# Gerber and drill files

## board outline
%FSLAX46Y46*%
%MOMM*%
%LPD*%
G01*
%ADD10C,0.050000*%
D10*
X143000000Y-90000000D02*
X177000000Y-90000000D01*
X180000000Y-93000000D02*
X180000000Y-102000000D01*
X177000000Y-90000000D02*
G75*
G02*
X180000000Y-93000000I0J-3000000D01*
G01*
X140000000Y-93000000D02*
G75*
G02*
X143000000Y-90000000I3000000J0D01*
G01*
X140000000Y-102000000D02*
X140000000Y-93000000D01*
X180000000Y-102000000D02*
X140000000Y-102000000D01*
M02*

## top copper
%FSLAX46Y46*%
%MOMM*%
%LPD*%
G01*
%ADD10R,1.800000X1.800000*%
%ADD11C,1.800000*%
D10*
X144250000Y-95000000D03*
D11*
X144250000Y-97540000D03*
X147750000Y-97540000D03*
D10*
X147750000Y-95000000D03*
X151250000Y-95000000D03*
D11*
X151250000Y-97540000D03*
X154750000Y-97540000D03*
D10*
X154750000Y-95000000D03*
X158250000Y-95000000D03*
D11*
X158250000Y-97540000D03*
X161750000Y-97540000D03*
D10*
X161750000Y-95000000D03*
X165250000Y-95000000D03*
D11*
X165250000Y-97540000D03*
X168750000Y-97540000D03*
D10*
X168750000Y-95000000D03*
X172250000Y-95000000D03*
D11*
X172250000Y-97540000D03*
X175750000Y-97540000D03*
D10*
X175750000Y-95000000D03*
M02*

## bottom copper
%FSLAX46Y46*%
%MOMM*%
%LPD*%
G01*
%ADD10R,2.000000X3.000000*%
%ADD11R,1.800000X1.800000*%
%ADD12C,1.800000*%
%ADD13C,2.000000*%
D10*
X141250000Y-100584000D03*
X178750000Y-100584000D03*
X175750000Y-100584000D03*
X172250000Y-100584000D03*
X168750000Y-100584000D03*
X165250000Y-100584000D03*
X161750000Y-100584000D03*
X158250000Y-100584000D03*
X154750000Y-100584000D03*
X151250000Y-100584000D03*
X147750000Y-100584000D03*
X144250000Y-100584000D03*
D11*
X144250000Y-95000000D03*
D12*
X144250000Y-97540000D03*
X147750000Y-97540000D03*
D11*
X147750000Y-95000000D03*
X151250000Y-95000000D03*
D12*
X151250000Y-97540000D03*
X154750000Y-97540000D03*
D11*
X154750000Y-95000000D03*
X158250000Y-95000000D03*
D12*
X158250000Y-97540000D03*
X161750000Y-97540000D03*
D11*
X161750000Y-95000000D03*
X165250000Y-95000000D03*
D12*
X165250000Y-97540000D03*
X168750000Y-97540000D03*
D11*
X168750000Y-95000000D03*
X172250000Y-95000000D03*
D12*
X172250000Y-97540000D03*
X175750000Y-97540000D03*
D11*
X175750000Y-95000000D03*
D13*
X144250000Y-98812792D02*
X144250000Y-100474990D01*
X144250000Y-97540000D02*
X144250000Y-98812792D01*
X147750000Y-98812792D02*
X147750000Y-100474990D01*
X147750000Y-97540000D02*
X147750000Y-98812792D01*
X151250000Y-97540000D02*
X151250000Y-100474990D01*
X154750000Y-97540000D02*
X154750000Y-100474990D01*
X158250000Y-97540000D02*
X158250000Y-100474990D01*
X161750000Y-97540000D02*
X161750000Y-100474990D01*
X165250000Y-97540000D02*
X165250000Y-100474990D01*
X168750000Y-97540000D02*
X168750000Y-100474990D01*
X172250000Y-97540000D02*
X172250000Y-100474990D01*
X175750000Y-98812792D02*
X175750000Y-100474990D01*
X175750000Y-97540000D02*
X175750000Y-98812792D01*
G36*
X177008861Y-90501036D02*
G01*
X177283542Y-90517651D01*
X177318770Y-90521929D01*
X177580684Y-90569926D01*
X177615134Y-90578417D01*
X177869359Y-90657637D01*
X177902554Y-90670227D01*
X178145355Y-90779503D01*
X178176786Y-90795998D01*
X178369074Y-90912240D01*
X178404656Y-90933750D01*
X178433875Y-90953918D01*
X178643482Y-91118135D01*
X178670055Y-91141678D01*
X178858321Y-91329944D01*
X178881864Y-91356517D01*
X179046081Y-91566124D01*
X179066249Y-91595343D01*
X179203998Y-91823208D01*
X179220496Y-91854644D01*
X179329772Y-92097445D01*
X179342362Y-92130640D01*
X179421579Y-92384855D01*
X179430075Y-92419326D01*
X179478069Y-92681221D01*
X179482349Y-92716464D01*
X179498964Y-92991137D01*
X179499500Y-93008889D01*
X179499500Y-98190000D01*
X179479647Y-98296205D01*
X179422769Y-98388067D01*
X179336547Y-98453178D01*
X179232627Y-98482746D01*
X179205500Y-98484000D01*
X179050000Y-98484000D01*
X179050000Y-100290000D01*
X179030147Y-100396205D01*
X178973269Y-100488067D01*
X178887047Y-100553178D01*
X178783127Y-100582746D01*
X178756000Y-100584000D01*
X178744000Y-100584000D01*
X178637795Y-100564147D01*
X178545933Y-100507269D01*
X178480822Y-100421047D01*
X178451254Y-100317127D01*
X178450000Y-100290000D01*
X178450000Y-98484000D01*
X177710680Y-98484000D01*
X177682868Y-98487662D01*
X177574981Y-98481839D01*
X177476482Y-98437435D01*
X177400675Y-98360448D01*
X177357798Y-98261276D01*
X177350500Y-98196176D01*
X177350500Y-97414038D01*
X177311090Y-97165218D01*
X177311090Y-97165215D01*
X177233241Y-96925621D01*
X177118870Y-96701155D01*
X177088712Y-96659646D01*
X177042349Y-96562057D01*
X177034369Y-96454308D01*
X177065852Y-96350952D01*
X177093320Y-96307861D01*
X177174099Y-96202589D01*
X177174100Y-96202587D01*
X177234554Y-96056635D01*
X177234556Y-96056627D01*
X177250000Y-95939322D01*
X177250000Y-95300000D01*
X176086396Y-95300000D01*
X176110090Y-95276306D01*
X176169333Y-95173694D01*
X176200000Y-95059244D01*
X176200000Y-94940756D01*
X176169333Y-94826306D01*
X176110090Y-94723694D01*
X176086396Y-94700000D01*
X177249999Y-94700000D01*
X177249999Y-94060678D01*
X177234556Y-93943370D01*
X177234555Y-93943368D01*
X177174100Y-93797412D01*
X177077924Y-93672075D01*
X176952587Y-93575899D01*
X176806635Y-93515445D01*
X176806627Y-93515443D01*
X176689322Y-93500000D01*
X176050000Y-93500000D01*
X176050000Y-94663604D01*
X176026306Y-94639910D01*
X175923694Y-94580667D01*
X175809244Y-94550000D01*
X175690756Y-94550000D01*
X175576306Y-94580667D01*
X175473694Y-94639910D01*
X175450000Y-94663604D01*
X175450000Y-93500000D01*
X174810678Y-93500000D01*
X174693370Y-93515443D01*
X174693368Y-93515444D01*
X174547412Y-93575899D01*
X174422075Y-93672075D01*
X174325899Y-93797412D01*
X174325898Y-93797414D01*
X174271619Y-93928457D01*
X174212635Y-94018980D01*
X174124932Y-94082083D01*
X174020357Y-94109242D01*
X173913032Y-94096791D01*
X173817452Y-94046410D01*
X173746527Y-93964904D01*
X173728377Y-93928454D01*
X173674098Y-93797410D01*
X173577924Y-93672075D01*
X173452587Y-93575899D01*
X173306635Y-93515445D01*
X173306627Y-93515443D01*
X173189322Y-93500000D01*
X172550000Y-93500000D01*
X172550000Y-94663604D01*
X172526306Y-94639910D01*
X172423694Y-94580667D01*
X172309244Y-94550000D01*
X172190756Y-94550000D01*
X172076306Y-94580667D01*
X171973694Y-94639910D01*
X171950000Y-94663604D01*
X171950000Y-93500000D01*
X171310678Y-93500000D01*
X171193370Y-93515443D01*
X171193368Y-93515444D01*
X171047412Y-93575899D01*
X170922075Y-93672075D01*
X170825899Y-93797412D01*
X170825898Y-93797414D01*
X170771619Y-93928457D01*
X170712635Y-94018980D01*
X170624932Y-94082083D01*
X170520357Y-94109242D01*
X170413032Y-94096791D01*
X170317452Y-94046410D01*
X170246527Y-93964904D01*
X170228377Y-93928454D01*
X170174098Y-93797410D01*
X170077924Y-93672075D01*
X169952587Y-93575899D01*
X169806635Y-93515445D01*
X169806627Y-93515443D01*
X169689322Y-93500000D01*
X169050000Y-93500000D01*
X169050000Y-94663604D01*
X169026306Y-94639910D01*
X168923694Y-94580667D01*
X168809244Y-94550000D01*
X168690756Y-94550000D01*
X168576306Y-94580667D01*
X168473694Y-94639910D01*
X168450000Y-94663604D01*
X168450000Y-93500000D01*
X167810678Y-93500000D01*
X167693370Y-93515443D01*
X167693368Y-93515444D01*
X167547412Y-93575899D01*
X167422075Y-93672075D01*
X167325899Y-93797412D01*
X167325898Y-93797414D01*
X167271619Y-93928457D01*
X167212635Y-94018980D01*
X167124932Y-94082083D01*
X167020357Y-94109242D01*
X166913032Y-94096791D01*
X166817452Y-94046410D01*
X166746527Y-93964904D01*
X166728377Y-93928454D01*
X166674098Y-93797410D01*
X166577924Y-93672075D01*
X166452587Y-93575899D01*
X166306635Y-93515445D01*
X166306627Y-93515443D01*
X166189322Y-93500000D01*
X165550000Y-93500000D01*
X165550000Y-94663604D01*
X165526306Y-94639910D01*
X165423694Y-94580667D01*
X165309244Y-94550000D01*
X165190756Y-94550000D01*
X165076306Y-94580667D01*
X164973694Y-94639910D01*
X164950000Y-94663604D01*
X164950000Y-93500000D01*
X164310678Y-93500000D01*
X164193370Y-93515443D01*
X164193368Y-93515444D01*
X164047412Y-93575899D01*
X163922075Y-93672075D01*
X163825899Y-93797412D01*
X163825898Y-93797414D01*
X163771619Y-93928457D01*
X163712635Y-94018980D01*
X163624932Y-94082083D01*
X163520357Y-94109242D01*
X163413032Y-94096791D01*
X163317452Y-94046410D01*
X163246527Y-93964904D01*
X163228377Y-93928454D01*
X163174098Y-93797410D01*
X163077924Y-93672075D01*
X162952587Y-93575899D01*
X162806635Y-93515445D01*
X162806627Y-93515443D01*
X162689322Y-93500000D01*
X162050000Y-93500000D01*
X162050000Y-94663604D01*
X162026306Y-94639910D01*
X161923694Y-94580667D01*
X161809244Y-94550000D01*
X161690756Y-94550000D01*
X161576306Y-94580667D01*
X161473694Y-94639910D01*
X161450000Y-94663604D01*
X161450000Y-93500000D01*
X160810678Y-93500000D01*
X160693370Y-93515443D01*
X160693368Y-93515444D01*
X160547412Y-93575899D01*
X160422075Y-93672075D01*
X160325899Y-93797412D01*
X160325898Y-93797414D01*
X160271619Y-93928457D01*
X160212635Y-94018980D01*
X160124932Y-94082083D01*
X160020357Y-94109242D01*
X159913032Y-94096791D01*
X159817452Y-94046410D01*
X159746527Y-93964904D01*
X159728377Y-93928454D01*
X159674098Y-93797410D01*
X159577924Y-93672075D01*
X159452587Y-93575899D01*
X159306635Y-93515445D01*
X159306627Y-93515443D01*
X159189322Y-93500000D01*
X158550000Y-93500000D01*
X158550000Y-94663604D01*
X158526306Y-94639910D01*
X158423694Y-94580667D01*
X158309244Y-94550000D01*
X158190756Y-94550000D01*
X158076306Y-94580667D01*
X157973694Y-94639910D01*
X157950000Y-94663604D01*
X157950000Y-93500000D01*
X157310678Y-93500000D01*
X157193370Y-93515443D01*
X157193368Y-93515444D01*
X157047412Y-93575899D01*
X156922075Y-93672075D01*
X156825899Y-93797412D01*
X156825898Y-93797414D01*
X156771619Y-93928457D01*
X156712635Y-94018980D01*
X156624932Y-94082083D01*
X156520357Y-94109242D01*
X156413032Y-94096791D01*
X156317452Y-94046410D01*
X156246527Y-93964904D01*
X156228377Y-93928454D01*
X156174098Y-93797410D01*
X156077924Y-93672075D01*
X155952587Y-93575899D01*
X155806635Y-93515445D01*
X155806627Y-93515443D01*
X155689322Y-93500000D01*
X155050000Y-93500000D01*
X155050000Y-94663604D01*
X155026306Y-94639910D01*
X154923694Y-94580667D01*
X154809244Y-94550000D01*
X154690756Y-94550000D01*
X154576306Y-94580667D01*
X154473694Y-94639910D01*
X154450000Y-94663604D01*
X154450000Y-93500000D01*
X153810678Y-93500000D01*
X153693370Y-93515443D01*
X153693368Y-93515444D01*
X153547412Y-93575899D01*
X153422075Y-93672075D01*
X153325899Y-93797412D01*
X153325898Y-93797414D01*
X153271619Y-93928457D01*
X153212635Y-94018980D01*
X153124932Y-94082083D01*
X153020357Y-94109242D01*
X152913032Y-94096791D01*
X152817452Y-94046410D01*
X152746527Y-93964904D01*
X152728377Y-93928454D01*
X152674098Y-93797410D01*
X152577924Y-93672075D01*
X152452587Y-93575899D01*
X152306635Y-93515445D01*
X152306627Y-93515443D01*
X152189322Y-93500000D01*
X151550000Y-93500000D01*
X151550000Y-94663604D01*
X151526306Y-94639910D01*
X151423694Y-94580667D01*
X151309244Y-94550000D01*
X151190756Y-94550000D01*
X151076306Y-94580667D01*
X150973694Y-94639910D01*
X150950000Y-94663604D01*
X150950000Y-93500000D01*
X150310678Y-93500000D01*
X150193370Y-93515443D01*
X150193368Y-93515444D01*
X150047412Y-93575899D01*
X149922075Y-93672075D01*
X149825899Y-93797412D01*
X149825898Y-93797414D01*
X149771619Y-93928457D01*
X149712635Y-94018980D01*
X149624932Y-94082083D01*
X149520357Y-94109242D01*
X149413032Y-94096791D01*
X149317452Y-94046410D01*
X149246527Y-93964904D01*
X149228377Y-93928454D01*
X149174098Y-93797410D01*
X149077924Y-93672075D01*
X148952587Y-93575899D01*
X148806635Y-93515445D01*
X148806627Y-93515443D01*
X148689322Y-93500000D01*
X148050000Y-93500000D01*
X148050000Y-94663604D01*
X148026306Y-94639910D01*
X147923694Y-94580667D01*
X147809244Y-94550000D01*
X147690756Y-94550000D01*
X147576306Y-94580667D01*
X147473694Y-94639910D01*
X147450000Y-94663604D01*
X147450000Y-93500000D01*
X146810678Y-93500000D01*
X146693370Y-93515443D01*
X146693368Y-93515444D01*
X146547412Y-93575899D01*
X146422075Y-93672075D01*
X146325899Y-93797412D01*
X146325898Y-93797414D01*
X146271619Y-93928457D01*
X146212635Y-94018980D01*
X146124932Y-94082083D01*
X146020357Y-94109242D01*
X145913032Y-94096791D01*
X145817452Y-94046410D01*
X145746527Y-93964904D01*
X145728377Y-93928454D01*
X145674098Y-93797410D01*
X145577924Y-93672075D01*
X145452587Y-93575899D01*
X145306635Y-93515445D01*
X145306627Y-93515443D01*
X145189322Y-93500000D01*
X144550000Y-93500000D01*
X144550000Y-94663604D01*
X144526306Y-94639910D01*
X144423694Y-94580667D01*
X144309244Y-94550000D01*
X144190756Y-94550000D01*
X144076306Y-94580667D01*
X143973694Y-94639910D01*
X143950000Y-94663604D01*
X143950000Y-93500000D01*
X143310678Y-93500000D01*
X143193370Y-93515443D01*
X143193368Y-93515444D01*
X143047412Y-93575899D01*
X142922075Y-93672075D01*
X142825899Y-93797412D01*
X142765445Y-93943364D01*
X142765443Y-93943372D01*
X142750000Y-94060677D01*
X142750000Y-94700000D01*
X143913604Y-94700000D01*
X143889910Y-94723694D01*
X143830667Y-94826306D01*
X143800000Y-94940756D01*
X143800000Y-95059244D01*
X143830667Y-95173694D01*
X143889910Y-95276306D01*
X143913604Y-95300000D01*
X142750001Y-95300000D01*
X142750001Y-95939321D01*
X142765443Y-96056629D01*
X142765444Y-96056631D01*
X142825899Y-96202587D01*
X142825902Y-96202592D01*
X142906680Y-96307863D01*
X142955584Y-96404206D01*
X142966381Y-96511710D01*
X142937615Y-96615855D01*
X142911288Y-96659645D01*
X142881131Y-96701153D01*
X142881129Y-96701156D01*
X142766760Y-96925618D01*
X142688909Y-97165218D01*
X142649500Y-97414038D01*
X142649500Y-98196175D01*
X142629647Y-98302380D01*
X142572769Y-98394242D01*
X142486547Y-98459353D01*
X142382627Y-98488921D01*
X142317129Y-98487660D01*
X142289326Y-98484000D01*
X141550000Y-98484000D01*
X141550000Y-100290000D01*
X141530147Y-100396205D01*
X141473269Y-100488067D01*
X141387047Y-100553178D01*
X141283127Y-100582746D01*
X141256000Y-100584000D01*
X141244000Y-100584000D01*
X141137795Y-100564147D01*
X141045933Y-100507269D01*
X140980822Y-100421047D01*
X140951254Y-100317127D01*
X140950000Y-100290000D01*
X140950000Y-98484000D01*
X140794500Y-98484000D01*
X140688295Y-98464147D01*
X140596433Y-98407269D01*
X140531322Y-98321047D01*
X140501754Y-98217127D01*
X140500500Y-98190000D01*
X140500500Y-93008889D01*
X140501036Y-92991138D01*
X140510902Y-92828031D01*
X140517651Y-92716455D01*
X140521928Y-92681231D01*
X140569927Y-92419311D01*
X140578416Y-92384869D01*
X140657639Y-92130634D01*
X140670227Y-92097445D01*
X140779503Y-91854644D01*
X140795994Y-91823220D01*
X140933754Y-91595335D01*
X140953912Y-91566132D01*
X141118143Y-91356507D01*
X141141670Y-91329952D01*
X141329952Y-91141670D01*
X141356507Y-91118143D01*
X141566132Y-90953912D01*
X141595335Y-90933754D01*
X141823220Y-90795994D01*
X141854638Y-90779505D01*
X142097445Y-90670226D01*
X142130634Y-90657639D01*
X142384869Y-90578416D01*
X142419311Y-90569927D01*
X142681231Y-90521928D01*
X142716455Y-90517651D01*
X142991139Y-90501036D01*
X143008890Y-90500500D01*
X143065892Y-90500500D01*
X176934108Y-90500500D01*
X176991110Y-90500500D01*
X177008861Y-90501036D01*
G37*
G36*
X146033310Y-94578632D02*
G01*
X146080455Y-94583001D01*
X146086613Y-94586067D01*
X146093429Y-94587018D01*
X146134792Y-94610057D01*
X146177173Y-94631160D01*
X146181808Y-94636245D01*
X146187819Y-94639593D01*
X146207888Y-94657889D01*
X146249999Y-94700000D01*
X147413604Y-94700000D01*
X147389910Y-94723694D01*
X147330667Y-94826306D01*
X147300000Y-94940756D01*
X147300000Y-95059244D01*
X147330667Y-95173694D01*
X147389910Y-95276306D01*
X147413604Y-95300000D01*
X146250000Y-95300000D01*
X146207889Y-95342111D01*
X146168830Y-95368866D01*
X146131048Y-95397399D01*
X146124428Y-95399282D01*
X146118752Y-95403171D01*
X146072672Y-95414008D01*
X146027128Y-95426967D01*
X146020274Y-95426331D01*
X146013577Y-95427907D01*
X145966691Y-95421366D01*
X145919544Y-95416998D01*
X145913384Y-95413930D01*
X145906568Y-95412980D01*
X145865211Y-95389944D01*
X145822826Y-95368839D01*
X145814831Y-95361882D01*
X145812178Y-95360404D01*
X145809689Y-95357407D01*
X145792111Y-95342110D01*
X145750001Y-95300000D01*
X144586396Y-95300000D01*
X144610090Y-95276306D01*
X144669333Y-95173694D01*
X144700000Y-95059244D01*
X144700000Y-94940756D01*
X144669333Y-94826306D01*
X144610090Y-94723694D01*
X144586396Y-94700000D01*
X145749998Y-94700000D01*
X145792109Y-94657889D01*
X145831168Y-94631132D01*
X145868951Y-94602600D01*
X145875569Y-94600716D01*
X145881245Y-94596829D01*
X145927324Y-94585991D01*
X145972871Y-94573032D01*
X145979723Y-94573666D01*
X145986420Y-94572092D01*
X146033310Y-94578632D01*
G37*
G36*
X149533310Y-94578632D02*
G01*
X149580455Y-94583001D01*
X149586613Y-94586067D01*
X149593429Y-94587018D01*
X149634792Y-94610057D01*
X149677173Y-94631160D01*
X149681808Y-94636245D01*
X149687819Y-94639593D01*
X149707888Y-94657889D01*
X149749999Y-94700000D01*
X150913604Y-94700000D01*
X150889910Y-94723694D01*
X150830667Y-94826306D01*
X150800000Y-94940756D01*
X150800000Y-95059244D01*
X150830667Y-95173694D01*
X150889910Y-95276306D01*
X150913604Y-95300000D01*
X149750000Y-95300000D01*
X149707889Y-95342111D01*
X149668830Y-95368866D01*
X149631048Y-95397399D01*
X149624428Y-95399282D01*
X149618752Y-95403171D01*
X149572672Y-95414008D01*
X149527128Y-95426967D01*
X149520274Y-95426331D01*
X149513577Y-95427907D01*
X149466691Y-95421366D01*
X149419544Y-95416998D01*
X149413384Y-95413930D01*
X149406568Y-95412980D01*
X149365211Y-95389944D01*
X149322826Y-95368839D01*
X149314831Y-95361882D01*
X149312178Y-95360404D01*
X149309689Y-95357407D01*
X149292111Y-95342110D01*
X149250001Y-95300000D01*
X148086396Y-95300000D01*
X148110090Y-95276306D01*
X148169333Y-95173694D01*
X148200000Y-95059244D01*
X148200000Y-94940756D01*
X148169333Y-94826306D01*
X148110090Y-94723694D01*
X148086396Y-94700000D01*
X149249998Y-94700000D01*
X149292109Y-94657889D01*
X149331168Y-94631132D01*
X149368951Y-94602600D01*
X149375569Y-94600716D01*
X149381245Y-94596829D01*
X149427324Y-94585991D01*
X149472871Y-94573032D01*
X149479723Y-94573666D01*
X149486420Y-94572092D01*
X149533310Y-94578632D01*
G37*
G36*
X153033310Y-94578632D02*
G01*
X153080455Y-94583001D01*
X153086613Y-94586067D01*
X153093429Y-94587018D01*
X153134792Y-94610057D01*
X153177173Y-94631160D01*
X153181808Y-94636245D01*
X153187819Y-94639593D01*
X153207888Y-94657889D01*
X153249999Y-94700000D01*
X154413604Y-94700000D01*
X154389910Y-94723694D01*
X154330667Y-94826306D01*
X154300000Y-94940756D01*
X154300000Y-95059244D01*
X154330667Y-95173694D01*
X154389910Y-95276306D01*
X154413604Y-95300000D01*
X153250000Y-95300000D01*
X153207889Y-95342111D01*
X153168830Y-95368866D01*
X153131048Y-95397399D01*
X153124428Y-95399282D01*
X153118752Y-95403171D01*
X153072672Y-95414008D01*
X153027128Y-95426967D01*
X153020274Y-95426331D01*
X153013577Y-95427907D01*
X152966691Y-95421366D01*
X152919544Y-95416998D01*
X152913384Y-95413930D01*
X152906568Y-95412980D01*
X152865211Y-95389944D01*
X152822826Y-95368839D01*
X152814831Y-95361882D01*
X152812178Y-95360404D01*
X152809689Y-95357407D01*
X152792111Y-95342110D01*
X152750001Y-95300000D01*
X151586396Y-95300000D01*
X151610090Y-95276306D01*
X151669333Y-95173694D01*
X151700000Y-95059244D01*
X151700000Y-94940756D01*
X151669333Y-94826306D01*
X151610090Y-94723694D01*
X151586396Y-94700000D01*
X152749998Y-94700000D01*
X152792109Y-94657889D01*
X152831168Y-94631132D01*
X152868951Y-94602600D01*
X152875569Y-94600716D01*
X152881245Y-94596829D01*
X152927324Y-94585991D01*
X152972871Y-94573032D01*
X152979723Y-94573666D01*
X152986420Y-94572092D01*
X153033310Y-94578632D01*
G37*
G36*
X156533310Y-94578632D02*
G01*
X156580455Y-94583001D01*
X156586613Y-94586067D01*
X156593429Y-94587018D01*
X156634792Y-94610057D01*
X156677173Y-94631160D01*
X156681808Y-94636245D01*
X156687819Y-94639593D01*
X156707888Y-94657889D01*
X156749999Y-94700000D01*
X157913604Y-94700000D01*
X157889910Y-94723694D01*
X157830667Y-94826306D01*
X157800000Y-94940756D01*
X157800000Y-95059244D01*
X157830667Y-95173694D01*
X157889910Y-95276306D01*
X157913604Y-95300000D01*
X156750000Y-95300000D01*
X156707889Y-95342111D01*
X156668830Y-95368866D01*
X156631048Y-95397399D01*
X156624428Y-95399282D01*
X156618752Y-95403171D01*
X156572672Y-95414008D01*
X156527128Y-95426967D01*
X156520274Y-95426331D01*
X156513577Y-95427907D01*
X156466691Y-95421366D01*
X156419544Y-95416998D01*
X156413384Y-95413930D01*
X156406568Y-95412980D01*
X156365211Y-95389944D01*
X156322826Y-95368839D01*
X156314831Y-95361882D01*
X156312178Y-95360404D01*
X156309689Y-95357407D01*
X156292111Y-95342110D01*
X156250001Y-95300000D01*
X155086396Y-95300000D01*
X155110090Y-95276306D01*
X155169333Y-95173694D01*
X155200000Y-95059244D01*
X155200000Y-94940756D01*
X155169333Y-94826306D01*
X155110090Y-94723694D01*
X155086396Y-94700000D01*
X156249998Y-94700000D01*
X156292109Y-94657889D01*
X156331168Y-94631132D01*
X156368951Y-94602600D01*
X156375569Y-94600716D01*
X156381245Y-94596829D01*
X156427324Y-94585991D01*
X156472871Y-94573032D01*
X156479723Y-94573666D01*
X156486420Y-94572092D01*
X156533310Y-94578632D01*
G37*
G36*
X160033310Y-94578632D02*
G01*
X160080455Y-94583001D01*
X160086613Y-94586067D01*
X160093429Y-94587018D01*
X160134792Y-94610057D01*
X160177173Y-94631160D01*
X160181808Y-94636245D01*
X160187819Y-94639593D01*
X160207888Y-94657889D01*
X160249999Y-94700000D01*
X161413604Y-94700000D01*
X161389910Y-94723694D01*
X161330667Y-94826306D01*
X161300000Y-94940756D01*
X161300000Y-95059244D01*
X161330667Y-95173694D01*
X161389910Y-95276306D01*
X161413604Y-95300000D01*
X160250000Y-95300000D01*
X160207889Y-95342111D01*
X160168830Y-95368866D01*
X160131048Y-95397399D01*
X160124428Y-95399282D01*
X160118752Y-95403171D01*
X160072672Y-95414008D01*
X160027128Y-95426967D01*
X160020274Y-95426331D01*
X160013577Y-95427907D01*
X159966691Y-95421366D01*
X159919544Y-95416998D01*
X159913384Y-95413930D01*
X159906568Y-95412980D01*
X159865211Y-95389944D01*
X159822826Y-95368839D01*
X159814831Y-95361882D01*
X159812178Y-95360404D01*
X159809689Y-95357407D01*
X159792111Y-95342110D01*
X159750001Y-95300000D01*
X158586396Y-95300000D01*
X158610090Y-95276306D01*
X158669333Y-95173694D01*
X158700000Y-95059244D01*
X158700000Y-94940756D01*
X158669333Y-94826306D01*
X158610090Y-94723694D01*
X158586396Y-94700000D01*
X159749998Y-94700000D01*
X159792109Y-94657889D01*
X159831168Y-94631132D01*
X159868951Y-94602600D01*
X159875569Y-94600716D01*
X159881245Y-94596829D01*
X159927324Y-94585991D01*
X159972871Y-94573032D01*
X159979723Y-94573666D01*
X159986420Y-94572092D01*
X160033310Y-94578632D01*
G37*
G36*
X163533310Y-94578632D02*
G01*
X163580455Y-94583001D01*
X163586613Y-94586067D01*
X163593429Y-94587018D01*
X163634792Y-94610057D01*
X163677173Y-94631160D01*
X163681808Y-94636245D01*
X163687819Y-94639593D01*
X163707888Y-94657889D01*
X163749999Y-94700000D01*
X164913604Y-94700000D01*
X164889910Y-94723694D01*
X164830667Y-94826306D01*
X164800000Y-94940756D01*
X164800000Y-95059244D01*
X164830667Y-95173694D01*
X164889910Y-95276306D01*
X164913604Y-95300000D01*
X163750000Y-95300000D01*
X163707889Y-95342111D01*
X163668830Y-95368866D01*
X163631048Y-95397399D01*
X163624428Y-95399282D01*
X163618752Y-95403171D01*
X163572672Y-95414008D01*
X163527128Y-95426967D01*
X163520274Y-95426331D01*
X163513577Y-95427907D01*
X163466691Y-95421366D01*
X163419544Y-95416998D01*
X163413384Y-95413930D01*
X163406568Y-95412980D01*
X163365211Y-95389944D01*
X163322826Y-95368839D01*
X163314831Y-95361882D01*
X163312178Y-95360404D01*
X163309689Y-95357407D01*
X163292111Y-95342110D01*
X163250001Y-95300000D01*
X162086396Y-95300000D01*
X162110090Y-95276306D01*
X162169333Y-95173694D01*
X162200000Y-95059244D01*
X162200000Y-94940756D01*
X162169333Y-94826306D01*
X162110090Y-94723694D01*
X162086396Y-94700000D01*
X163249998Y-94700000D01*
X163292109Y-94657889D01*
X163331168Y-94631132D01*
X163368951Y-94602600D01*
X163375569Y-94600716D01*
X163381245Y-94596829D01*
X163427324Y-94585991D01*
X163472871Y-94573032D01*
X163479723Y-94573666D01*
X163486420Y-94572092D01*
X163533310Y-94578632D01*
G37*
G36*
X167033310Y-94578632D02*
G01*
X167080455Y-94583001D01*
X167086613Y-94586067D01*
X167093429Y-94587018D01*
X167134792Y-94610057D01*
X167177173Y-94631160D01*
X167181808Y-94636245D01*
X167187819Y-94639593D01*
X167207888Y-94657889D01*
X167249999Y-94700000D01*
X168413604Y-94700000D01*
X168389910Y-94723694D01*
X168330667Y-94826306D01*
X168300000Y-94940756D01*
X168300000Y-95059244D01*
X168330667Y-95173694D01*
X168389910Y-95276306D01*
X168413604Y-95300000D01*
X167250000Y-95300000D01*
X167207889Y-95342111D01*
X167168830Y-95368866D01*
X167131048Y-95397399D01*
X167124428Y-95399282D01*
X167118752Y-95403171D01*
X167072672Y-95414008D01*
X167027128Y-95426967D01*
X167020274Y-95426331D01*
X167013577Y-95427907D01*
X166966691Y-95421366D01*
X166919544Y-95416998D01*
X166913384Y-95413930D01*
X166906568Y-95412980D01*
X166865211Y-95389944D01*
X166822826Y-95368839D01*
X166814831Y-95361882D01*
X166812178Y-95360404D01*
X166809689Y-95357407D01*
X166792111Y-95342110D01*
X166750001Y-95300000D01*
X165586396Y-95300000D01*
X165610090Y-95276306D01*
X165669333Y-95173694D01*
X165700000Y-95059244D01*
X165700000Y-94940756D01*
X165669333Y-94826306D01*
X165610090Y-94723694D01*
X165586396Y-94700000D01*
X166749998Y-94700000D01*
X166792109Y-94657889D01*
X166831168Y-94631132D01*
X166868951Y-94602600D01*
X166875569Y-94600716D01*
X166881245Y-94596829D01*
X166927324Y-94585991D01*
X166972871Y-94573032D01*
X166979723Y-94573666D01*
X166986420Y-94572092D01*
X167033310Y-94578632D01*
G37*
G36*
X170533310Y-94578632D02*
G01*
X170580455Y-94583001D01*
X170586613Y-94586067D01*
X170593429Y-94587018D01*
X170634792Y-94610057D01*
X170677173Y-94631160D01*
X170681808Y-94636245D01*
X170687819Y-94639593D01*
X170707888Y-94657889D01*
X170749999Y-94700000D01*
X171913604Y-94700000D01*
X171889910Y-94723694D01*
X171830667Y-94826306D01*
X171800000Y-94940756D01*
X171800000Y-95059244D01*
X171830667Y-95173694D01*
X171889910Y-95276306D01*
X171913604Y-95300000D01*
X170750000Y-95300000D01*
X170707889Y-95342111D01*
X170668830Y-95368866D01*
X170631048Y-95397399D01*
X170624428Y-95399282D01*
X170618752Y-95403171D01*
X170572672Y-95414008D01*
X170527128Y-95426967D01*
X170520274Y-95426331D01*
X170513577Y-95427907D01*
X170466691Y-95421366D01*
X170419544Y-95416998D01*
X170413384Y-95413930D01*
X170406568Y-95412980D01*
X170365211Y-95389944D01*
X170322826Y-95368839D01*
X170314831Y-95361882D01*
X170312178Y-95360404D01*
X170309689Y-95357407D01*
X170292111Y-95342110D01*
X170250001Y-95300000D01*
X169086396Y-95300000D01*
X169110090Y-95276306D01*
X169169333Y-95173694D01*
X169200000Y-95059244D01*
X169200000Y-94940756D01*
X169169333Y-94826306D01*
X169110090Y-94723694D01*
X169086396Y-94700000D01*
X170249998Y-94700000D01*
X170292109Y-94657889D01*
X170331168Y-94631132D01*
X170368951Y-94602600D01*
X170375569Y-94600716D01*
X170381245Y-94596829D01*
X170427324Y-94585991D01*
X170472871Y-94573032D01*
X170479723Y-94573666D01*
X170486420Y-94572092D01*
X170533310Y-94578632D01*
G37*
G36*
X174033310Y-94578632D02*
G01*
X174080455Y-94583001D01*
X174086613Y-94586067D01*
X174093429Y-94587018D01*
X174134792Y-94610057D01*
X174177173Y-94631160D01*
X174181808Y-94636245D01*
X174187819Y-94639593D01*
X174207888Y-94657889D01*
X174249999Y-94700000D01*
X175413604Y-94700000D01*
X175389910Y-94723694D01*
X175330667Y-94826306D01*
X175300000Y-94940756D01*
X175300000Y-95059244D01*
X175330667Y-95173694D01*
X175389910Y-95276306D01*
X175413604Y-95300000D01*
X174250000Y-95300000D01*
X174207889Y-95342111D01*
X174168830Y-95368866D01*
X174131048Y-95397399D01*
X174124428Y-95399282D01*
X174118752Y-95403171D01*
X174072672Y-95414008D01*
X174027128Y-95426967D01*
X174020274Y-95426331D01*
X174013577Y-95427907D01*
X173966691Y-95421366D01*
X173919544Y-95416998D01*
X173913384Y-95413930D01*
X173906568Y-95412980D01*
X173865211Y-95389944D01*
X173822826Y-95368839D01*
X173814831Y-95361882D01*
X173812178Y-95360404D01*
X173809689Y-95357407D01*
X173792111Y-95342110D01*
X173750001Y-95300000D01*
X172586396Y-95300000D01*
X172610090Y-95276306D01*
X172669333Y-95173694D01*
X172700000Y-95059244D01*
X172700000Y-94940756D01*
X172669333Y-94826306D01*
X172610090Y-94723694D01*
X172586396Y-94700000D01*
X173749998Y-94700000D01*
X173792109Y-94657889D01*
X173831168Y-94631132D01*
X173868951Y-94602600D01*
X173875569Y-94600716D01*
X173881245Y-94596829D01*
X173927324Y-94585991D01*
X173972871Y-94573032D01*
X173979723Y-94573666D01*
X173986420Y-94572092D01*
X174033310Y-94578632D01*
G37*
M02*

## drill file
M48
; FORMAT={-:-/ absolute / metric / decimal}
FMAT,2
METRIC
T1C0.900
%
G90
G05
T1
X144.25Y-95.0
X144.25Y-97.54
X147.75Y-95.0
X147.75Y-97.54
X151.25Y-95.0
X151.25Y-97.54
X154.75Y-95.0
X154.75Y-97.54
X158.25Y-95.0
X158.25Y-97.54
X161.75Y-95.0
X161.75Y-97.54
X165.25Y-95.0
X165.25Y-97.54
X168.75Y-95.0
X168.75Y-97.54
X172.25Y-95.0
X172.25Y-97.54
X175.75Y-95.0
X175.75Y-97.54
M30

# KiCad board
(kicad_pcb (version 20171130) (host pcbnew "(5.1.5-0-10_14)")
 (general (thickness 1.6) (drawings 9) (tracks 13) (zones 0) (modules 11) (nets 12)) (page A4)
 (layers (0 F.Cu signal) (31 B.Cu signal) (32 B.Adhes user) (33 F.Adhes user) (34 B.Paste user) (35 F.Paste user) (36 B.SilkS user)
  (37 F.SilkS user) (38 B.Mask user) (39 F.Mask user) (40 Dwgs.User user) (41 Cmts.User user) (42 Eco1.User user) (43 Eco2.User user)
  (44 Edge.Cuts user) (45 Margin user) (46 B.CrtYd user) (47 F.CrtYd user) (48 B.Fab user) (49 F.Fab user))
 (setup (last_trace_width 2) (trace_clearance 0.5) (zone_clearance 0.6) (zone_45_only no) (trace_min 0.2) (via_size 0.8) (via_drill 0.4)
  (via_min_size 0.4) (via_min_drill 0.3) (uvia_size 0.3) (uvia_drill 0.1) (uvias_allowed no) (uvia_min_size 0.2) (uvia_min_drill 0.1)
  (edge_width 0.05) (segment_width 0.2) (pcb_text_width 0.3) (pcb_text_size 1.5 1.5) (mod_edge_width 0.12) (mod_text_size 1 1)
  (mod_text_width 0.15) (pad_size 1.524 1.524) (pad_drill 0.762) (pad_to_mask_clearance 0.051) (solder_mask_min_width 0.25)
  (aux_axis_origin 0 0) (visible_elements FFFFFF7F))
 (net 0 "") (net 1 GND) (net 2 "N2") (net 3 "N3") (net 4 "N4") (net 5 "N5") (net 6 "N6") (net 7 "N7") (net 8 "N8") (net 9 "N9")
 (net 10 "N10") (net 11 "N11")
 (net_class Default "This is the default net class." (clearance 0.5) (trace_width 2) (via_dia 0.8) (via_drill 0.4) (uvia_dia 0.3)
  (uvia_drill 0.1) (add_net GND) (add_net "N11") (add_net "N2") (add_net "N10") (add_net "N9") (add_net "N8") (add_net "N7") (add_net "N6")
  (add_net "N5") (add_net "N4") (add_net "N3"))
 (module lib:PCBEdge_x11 (layer B.Cu) (at 144.25 100.584)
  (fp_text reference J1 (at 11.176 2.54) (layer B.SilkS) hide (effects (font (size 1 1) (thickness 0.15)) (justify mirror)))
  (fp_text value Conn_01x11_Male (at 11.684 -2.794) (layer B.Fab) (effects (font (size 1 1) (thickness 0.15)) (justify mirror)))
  (pad 11 connect rect (at -3 0) (size 2 3) (layers B.Cu B.Mask) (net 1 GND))
  (pad 11 connect rect (at 34.5 0) (size 2 3) (layers B.Cu B.Mask) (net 1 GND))
  (pad 10 connect rect (at 31.5 0) (size 2 3) (layers B.Cu B.Mask) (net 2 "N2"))
  (pad 9 connect rect (at 28 0) (size 2 3) (layers B.Cu B.Mask) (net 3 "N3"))
  (pad 8 connect rect (at 24.5 0) (size 2 3) (layers B.Cu B.Mask) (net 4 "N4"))
  (pad 7 connect rect (at 21 0) (size 2 3) (layers B.Cu B.Mask) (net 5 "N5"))
  (pad 6 connect rect (at 17.5 0 180) (size 2 3) (layers B.Cu B.Mask) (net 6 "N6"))
  (pad 5 connect rect (at 14 0) (size 2 3) (layers B.Cu B.Mask) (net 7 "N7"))
  (pad 4 connect rect (at 10.5 0) (size 2 3) (layers B.Cu B.Mask) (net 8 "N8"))
  (pad 3 connect rect (at 7 0) (size 2 3) (layers B.Cu B.Mask) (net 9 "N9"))
  (pad 2 connect rect (at 3.5 0) (size 2 3) (layers B.Cu B.Mask) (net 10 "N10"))
  (pad 1 connect rect (at 0 0) (size 2 3) (layers B.Cu B.Mask) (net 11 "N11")))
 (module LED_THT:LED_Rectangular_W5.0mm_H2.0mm (layer F.Cu) (at 144.25 95 270)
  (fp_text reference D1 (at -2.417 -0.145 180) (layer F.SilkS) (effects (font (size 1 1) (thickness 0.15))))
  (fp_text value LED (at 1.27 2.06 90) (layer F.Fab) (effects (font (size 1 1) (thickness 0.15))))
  (pad 1 thru_hole rect (at 0 0 270) (size 1.8 1.8) (drill 0.9) (layers *.Cu *.Mask) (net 1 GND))
  (pad 2 thru_hole circle (at 2.54 0 270) (size 1.8 1.8) (drill 0.9) (layers *.Cu *.Mask) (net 11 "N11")))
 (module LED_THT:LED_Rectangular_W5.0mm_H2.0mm (layer F.Cu) (at 147.75 95 270)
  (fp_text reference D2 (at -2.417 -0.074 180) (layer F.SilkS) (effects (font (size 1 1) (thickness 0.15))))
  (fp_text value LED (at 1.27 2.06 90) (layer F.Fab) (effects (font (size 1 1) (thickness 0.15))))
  (pad 2 thru_hole circle (at 2.54 0 270) (size 1.8 1.8) (drill 0.9) (layers *.Cu *.Mask) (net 10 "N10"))
  (pad 1 thru_hole rect (at 0 0 270) (size 1.8 1.8) (drill 0.9) (layers *.Cu *.Mask) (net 1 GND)))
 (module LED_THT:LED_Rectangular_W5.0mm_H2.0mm (layer F.Cu) (at 151.25 95 270)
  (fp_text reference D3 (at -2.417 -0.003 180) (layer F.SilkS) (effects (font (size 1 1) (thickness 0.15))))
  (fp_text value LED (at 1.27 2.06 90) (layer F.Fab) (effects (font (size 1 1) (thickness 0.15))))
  (pad 1 thru_hole rect (at 0 0 270) (size 1.8 1.8) (drill 0.9) (layers *.Cu *.Mask) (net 1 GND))
  (pad 2 thru_hole circle (at 2.54 0 270) (size 1.8 1.8) (drill 0.9) (layers *.Cu *.Mask) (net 9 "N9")))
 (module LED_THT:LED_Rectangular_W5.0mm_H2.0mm (layer F.Cu) (at 154.75 95 270)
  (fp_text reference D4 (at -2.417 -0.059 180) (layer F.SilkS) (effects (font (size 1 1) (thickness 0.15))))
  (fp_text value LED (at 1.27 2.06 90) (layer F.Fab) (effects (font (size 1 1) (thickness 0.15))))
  (pad 2 thru_hole circle (at 2.54 0 270) (size 1.8 1.8) (drill 0.9) (layers *.Cu *.Mask) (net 8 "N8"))
  (pad 1 thru_hole rect (at 0 0 270) (size 1.8 1.8) (drill 0.9) (layers *.Cu *.Mask) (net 1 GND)))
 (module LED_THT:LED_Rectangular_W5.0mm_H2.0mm (layer F.Cu) (at 158.25 95 270)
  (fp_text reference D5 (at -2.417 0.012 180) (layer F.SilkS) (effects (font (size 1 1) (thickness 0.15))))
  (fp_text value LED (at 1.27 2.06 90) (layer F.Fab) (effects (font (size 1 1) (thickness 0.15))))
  (pad 1 thru_hole rect (at 0 0 270) (size 1.8 1.8) (drill 0.9) (layers *.Cu *.Mask) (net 1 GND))
  (pad 2 thru_hole circle (at 2.54 0 270) (size 1.8 1.8) (drill 0.9) (layers *.Cu *.Mask) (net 7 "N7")))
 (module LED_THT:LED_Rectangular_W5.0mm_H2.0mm (layer F.Cu) (at 161.75 95 270)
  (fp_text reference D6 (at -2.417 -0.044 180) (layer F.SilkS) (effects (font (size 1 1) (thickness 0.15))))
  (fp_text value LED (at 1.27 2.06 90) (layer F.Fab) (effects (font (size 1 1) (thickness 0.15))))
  (pad 2 thru_hole circle (at 2.54 0 270) (size 1.8 1.8) (drill 0.9) (layers *.Cu *.Mask) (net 6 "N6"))
  (pad 1 thru_hole rect (at 0 0 270) (size 1.8 1.8) (drill 0.9) (layers *.Cu *.Mask) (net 1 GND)))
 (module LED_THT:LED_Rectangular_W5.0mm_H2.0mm (layer F.Cu) (at 165.25 95 270)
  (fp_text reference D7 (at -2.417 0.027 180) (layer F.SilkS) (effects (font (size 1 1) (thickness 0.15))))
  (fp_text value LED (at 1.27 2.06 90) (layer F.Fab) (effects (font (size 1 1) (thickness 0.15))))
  (pad 1 thru_hole rect (at 0 0 270) (size 1.8 1.8) (drill 0.9) (layers *.Cu *.Mask) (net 1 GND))
  (pad 2 thru_hole circle (at 2.54 0 270) (size 1.8 1.8) (drill 0.9) (layers *.Cu *.Mask) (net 5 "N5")))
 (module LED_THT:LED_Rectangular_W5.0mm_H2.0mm (layer F.Cu) (at 168.75 95 270)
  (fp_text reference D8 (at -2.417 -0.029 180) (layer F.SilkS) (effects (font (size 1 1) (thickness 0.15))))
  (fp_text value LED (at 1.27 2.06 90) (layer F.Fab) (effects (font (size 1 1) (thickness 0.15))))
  (pad 2 thru_hole circle (at 2.54 0 270) (size 1.8 1.8) (drill 0.9) (layers *.Cu *.Mask) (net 4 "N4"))
  (pad 1 thru_hole rect (at 0 0 270) (size 1.8 1.8) (drill 0.9) (layers *.Cu *.Mask) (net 1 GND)))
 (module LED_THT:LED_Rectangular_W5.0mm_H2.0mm (layer F.Cu) (at 172.25 95 270)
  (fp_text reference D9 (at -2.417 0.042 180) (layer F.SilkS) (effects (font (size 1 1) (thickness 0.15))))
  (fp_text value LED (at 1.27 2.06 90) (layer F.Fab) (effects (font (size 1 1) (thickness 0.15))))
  (pad 1 thru_hole rect (at 0 0 270) (size 1.8 1.8) (drill 0.9) (layers *.Cu *.Mask) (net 1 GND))
  (pad 2 thru_hole circle (at 2.54 0 270) (size 1.8 1.8) (drill 0.9) (layers *.Cu *.Mask) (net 3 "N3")))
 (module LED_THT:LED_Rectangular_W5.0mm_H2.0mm (layer F.Cu) (at 175.75 95 270)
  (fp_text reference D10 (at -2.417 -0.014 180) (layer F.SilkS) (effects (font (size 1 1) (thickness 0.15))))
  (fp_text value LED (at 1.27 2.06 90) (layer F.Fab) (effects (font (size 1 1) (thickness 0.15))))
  (pad 2 thru_hole circle (at 2.54 0 270) (size 1.8 1.8) (drill 0.9) (layers *.Cu *.Mask) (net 2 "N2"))
  (pad 1 thru_hole rect (at 0 0 270) (size 1.8 1.8) (drill 0.9) (layers *.Cu *.Mask) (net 1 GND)))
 (gr_line (start 143 90) (end 177 90) (layer Edge.Cuts) (width 0.05))
 (gr_line (start 180 93) (end 180 102) (layer Edge.Cuts) (width 0.05))
 (gr_arc (start 177 93) (end 180 93) (angle -90) (layer Edge.Cuts) (width 0.05))
 (gr_arc (start 143 93) (end 143 90) (angle -90) (layer Edge.Cuts) (width 0.05))
 (gr_line (start 140 102) (end 140 93) (layer Edge.Cuts) (width 0.05))
 (gr_line (start 180 102) (end 140 102) (layer Edge.Cuts) (width 0.05))
 (segment (start 144.25 98.812792) (end 144.25 100.47499) (width 2) (layer B.Cu) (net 11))
 (segment (start 144.25 97.54) (end 144.25 98.812792) (width 2) (layer B.Cu) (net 11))
 (segment (start 147.75 98.812792) (end 147.75 100.47499) (width 2) (layer B.Cu) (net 10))
 (segment (start 147.75 97.54) (end 147.75 98.812792) (width 2) (layer B.Cu) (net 10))
 (segment (start 151.25 97.54) (end 151.25 100.47499) (width 2) (layer B.Cu) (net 9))
 (segment (start 154.75 97.54) (end 154.75 100.47499) (width 2) (layer B.Cu) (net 8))
 (segment (start 158.25 97.54) (end 158.25 100.47499) (width 2) (layer B.Cu) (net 7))
 (segment (start 161.75 97.54) (end 161.75 100.47499) (width 2) (layer B.Cu) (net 6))
 (segment (start 165.25 97.54) (end 165.25 100.47499) (width 2) (layer B.Cu) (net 5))
 (segment (start 168.75 97.54) (end 168.75 100.47499) (width 2) (layer B.Cu) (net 4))
 (segment (start 172.25 97.54) (end 172.25 100.47499) (width 2) (layer B.Cu) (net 3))
 (segment (start 175.75 98.812792) (end 175.75 100.47499) (width 2) (layer B.Cu) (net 2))
 (segment (start 175.75 97.54) (end 175.75 98.812792) (width 2) (layer B.Cu) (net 2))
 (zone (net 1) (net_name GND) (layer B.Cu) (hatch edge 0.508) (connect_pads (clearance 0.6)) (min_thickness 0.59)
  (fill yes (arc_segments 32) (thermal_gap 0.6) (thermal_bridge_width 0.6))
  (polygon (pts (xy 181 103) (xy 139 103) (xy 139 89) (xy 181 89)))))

